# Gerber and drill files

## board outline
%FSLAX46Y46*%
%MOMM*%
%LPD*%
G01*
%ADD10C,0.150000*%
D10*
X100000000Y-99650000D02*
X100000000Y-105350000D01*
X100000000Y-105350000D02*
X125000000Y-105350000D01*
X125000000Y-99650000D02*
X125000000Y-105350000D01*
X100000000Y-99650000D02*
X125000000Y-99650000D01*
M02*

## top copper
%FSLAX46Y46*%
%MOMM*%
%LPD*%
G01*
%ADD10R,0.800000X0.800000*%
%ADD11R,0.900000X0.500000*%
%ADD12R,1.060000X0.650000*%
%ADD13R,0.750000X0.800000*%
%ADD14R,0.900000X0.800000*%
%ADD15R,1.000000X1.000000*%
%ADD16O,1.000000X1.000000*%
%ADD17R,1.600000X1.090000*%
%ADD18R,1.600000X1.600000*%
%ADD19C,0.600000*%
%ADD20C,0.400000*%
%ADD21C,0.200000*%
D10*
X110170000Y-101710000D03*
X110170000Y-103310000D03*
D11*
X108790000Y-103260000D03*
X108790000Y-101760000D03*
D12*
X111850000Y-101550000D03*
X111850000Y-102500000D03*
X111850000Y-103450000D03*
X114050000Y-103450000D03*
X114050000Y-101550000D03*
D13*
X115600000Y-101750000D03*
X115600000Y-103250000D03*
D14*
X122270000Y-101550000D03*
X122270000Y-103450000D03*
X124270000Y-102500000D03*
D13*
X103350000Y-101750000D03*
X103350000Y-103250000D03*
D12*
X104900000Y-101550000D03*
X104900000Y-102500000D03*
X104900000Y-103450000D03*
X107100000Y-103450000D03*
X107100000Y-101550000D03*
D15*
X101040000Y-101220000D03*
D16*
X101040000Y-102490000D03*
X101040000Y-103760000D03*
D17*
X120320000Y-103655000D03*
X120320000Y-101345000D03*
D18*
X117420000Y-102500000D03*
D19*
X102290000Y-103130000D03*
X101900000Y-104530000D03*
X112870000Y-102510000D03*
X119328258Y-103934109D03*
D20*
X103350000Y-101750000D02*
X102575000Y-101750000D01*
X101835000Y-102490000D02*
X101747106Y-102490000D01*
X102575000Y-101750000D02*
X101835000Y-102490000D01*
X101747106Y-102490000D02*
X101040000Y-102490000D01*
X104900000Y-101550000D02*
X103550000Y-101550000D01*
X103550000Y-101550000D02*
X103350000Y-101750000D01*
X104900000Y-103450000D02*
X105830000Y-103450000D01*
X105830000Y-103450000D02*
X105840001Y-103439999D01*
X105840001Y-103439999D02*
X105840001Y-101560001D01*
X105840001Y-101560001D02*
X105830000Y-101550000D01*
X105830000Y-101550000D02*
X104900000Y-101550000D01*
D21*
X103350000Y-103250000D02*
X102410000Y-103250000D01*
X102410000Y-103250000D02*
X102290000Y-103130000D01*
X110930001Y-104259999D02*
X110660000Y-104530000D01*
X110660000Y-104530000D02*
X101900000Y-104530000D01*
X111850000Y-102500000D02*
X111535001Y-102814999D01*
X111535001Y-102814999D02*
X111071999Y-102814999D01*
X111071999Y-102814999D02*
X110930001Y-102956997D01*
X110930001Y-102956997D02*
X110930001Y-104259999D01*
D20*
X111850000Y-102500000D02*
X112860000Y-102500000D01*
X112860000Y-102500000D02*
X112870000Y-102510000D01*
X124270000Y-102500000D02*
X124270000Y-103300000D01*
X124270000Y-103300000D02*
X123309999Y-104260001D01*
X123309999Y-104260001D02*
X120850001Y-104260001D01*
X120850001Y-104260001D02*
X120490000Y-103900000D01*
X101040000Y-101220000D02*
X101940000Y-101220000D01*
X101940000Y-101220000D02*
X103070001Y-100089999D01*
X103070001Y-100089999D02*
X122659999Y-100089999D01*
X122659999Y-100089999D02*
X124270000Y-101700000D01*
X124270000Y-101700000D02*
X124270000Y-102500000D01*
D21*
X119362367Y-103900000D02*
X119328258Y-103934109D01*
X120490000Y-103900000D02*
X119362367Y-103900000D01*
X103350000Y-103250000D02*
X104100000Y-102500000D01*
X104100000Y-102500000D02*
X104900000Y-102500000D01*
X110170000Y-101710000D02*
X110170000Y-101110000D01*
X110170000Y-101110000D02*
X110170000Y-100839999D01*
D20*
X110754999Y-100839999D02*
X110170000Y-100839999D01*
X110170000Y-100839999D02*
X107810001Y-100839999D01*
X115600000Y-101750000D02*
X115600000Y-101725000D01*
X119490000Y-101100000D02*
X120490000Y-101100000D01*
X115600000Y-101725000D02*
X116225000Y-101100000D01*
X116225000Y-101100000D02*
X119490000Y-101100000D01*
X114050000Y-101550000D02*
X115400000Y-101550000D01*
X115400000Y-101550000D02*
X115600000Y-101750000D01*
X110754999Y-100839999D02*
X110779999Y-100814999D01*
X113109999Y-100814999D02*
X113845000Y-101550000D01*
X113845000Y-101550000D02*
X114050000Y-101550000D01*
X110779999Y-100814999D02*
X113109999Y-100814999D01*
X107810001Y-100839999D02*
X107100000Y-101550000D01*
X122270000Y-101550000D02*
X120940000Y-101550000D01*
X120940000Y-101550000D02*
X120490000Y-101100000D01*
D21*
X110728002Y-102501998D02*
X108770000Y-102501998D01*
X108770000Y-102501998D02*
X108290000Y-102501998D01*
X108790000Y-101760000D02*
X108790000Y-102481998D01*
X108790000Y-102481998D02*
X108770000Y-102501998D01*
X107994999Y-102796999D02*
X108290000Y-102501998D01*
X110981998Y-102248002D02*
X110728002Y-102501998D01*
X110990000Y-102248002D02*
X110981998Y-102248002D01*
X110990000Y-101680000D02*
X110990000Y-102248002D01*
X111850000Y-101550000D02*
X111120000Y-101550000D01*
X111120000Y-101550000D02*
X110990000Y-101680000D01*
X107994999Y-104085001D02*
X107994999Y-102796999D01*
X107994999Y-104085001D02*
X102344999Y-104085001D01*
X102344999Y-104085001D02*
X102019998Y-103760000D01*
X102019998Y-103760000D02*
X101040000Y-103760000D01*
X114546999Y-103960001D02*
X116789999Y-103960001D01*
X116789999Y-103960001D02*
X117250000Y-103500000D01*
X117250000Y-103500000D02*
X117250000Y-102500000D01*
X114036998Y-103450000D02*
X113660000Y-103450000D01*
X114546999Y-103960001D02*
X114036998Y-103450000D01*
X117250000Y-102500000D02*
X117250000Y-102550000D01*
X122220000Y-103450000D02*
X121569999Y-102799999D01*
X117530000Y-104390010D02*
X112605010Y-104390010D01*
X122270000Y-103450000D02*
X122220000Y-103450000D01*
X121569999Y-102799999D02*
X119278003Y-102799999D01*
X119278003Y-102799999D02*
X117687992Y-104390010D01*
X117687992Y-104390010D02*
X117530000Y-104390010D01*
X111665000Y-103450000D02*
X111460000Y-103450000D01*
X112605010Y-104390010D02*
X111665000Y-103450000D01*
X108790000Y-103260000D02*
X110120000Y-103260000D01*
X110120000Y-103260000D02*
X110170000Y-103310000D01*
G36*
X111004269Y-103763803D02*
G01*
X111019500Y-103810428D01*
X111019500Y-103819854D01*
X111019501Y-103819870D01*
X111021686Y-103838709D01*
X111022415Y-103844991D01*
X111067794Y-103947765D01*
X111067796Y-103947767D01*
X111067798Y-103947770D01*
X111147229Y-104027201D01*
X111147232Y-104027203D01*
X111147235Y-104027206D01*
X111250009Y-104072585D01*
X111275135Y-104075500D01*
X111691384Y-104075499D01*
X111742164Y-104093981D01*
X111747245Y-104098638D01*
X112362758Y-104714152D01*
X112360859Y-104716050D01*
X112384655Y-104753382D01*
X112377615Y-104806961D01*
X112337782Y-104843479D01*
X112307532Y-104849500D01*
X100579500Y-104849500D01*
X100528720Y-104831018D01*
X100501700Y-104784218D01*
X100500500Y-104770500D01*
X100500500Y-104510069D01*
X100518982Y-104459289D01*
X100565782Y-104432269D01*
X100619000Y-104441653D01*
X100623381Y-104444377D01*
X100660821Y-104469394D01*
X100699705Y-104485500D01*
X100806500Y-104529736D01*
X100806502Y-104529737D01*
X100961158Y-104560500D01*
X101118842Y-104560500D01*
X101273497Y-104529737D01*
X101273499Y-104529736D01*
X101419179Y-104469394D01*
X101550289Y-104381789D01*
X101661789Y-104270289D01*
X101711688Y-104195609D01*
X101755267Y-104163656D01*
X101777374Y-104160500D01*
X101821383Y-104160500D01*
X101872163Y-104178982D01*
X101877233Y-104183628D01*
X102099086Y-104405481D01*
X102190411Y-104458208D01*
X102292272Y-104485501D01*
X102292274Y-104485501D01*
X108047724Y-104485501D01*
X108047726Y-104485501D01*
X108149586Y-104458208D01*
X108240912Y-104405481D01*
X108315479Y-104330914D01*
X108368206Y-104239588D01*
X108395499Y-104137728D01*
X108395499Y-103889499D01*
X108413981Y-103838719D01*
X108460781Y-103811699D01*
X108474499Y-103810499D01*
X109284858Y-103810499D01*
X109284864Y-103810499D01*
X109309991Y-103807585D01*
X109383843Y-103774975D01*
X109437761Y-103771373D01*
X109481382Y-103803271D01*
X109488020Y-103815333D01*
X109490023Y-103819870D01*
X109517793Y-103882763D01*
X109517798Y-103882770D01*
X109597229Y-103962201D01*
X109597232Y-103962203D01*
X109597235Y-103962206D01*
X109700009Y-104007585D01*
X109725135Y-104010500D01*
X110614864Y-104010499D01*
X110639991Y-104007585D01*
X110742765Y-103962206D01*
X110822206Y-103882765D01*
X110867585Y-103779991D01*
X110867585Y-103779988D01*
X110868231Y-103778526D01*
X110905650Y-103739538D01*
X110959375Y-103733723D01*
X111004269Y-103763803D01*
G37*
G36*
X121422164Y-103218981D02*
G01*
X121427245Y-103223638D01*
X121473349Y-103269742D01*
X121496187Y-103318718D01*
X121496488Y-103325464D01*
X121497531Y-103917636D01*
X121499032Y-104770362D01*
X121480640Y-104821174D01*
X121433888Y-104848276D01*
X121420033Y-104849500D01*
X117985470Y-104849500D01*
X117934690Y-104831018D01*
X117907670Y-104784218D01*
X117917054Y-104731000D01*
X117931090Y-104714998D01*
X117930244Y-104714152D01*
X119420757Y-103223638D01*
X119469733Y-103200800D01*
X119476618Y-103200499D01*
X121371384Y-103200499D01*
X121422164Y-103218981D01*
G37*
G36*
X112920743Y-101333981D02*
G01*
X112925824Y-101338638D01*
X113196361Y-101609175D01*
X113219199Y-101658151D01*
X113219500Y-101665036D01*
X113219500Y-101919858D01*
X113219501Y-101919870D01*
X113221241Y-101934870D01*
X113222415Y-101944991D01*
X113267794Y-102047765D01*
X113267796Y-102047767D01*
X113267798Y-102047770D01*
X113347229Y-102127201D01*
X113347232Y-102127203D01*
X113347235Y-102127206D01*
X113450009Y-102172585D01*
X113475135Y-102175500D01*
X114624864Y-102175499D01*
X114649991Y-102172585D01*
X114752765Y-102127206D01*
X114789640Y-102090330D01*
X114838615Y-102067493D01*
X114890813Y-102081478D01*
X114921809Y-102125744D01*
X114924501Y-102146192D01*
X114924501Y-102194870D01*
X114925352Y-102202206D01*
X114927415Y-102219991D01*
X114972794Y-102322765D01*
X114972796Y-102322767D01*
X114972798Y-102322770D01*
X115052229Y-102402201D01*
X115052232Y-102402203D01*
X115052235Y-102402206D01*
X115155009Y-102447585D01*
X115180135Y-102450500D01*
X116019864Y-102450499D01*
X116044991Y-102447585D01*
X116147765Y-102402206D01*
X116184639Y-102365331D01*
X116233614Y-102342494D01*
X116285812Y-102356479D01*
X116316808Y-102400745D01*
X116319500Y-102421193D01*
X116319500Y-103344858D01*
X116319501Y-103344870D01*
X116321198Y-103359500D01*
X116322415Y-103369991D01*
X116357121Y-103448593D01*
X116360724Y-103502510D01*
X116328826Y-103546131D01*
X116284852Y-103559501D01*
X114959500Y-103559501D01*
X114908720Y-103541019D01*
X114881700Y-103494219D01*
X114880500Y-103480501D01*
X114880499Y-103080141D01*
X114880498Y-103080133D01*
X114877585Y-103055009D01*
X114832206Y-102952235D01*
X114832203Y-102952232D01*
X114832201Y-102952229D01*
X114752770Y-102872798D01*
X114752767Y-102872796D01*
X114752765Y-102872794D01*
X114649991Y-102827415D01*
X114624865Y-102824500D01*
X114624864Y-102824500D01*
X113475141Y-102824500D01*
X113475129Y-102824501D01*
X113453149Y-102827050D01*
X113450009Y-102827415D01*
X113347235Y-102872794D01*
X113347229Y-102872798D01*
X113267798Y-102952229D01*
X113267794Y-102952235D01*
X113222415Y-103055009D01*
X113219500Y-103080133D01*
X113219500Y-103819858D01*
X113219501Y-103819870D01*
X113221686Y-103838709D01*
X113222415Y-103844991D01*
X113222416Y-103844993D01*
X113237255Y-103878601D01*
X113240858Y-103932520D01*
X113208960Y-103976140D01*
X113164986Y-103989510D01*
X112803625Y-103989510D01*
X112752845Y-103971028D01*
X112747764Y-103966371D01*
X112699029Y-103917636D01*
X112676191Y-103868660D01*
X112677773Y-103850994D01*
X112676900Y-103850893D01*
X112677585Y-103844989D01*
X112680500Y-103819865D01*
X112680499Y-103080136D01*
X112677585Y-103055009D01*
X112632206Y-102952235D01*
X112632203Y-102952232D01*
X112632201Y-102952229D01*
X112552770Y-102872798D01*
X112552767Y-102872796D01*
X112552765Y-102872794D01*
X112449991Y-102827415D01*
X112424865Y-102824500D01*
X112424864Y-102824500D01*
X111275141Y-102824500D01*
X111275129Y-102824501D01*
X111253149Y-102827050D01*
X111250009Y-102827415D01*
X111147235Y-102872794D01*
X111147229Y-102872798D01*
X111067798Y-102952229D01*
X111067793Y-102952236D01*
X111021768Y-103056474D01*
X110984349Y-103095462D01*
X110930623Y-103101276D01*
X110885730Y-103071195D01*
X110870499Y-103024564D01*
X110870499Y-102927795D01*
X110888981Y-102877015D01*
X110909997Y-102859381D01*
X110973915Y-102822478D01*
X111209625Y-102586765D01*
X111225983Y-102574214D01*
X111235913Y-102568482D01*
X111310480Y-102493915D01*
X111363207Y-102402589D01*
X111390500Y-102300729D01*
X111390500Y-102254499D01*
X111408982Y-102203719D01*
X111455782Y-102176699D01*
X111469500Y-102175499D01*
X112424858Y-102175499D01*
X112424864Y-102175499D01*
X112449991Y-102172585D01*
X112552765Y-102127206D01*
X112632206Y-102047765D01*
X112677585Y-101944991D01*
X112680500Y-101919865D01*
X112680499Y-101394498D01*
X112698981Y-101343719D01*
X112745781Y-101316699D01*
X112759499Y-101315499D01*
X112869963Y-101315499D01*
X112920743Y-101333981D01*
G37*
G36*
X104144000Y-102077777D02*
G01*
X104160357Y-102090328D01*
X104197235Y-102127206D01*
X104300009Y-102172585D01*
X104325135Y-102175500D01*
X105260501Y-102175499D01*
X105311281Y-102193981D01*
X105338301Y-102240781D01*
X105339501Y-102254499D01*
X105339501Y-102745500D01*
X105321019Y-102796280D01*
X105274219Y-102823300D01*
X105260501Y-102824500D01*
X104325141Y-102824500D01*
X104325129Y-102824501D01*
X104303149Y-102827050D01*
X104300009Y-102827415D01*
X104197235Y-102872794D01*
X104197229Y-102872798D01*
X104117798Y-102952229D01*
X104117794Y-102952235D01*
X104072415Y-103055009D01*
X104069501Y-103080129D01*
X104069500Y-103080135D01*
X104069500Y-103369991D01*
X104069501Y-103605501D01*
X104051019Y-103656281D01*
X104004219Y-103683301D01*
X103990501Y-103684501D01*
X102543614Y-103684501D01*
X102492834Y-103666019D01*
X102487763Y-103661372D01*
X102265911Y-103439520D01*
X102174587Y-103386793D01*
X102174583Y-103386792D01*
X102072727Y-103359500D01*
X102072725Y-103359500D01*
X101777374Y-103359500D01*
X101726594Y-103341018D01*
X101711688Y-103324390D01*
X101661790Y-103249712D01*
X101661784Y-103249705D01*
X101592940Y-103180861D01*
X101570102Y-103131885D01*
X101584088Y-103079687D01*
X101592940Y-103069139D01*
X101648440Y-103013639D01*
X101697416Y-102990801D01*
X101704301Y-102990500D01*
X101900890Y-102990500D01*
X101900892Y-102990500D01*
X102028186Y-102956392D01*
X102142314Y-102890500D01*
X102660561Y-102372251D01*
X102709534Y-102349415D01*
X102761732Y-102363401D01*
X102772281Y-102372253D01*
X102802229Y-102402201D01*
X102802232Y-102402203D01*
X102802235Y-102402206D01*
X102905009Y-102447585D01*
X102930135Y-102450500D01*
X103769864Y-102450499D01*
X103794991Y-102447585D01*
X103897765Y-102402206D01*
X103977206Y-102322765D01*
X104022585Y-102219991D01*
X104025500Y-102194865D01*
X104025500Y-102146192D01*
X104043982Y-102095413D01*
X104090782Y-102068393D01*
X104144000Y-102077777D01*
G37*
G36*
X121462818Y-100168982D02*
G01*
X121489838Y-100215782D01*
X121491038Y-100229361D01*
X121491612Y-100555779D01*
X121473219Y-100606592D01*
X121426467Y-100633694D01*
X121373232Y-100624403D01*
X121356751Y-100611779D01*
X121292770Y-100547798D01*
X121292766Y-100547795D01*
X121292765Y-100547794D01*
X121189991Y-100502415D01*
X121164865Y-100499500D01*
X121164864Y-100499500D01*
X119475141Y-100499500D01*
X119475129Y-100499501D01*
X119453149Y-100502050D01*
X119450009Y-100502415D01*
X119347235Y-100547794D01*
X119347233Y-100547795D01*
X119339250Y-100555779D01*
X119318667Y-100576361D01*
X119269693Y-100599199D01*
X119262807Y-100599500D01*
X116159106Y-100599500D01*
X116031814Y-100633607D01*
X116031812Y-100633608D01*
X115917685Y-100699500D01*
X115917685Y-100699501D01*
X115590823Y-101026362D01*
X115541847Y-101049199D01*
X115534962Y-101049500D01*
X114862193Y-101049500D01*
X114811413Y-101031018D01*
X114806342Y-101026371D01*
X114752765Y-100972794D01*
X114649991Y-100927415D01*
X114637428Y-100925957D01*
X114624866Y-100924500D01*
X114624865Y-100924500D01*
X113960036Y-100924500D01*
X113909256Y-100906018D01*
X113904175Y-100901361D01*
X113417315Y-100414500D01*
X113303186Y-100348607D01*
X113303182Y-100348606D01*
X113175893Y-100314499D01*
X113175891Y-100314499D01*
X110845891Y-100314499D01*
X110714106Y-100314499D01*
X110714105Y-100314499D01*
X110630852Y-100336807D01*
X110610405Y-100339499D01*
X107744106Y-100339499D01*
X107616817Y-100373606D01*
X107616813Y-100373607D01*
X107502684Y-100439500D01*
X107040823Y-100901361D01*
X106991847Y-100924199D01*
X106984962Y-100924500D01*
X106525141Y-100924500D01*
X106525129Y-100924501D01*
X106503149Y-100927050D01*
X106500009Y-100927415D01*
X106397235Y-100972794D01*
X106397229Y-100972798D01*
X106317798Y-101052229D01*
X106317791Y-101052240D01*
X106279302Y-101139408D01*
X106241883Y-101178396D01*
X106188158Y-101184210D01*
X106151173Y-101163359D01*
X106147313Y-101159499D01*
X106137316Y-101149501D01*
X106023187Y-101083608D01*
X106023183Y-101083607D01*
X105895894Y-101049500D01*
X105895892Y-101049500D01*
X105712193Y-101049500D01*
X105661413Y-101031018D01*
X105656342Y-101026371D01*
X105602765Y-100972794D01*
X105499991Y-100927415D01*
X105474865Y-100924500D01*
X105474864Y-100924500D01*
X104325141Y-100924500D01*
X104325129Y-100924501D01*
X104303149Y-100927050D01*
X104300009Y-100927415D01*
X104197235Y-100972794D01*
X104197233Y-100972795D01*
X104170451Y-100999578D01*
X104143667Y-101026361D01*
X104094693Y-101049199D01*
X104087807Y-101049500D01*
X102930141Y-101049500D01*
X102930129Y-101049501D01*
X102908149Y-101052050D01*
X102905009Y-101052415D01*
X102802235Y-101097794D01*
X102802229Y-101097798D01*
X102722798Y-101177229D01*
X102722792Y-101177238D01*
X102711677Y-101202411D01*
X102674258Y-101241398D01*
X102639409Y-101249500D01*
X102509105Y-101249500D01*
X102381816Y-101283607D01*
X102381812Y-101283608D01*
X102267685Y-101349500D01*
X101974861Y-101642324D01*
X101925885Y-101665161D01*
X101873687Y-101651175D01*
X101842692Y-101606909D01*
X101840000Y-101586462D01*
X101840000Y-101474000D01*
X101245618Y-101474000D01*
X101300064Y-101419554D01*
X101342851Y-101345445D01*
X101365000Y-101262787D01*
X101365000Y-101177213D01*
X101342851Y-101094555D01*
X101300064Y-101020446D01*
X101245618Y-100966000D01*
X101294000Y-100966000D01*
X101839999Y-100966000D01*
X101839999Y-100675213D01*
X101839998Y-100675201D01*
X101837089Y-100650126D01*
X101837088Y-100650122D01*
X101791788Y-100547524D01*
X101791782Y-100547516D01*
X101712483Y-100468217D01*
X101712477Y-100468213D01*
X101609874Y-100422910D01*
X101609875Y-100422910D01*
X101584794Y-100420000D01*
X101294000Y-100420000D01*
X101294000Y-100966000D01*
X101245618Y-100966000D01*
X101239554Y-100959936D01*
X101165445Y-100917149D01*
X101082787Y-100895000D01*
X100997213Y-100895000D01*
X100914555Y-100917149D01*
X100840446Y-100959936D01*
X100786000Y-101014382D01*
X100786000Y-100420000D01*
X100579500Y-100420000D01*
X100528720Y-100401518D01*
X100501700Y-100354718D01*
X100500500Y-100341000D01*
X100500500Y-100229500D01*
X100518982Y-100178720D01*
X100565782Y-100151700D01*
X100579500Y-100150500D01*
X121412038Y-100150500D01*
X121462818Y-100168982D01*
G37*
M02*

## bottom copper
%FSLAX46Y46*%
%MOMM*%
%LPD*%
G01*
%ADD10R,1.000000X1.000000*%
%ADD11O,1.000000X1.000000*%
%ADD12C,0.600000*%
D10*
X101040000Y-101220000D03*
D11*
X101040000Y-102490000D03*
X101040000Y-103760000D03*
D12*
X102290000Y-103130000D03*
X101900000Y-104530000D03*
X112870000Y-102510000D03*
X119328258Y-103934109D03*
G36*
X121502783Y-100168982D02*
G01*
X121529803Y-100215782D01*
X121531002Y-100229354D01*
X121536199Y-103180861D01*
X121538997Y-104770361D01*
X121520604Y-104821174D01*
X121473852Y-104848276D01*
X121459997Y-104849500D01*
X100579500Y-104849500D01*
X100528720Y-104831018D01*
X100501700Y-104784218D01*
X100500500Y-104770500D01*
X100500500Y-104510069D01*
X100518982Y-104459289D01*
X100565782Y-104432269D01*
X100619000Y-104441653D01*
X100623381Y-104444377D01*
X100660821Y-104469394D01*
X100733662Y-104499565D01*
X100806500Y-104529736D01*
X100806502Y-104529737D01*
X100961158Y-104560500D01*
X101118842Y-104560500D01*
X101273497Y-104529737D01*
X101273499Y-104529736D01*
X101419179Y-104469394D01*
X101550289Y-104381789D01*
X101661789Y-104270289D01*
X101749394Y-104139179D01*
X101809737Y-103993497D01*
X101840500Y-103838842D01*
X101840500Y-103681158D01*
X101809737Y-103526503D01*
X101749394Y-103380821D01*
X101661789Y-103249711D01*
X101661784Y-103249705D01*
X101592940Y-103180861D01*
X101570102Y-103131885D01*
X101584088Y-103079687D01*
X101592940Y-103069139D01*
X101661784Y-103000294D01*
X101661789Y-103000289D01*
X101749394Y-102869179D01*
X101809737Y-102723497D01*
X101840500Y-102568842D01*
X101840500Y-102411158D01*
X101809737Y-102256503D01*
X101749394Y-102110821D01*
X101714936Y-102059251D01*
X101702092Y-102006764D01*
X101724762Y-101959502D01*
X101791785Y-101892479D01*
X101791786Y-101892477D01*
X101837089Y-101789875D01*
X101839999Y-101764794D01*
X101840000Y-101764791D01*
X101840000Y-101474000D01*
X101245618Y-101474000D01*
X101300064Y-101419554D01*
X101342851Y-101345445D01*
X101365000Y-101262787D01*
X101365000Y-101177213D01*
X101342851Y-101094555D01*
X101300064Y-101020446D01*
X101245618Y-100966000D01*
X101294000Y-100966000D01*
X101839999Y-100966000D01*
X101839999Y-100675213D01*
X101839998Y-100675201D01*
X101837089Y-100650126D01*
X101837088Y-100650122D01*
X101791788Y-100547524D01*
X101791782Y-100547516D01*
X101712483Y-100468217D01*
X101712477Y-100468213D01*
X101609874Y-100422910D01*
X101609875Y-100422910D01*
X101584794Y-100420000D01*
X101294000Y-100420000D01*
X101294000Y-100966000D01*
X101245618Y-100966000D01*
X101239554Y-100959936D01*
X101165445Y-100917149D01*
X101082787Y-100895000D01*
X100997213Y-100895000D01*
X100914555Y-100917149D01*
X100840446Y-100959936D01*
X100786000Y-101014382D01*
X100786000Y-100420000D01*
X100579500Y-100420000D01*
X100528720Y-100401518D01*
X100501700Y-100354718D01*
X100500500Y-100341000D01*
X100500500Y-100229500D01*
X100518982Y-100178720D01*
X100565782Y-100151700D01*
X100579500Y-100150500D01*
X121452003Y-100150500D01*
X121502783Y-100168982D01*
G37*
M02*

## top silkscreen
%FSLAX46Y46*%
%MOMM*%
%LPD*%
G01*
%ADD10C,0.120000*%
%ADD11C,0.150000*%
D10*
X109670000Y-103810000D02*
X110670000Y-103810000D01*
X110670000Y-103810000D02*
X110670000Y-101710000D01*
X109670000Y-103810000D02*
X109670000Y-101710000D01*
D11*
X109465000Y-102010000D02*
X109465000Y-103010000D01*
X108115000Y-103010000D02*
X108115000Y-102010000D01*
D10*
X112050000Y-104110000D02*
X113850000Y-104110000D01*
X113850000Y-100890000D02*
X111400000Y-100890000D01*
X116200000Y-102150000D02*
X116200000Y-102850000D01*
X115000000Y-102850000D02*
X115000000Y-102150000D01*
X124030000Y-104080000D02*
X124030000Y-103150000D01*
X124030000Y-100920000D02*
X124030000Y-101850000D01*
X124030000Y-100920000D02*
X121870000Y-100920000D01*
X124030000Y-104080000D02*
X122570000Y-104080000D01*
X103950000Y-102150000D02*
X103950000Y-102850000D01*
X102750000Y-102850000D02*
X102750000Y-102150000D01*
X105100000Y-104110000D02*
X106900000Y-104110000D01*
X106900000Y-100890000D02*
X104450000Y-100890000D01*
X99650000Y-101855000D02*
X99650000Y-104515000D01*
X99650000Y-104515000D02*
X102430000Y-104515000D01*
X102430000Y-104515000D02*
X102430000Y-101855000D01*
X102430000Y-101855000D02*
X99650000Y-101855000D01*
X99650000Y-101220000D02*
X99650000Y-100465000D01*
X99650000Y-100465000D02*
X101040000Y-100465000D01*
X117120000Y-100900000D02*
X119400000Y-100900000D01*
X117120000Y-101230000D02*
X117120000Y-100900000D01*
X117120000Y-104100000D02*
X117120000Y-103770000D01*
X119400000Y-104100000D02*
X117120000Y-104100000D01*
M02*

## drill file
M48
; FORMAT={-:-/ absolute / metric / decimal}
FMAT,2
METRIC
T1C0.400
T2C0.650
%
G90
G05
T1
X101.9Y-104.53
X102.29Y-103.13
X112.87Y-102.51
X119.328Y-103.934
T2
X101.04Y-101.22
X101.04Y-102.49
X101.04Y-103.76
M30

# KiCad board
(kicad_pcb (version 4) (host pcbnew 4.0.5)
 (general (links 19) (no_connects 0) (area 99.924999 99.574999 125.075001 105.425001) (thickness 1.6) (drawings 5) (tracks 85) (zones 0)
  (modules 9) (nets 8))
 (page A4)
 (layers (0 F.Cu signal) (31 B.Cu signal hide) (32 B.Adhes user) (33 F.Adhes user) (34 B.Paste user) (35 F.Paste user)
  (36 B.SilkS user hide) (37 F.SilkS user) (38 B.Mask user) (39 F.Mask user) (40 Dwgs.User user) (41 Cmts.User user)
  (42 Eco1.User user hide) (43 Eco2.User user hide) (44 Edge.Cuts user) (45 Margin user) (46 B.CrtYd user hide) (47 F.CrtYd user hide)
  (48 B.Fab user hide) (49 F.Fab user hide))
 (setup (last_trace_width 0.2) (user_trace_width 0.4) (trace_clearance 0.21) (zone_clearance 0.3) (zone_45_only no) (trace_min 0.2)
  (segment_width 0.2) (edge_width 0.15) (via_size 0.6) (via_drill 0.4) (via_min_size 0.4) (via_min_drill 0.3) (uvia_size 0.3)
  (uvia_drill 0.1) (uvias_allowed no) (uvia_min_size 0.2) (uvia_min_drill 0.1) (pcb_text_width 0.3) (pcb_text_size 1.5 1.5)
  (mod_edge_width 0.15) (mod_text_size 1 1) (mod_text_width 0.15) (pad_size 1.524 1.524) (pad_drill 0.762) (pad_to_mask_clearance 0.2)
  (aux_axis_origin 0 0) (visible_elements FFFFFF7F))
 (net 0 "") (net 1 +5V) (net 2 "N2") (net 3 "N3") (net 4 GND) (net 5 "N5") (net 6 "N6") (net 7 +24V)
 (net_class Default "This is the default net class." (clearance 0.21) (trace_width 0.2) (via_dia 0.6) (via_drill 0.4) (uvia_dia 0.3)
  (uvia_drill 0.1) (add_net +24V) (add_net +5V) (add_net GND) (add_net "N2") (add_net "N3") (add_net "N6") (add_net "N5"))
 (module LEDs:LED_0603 (layer F.Cu) (at 110.17 102.51 90)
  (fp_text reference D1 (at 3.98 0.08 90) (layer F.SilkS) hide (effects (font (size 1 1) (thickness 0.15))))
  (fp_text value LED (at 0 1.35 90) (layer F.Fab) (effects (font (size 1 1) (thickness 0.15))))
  (fp_line (start -1.3 -0.5) (end -1.3 0.5) (layer F.SilkS) (width 0.12))
  (fp_line (start -1.3 0.5) (end 0.8 0.5) (layer F.SilkS) (width 0.12))
  (fp_line (start -1.3 -0.5) (end 0.8 -0.5) (layer F.SilkS) (width 0.12))
  (pad 2 smd rect (at 0.8 0 270) (size 0.8 0.8) (layers F.Cu F.Paste F.Mask) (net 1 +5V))
  (pad 1 smd rect (at -0.8 0 270) (size 0.8 0.8) (layers F.Cu F.Paste F.Mask) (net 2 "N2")))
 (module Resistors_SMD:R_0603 (layer F.Cu) (at 108.79 102.51 90)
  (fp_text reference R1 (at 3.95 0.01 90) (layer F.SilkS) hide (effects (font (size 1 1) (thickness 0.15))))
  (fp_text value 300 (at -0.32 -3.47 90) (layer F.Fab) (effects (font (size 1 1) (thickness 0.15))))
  (fp_line (start 0.5 0.675) (end -0.5 0.675) (layer F.SilkS) (width 0.15))
  (fp_line (start -0.5 -0.675) (end 0.5 -0.675) (layer F.SilkS) (width 0.15))
  (pad 1 smd rect (at -0.75 0 90) (size 0.5 0.9) (layers F.Cu F.Paste F.Mask) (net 2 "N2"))
  (pad 2 smd rect (at 0.75 0 90) (size 0.5 0.9) (layers F.Cu F.Paste F.Mask) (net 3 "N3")))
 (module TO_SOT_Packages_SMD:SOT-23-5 (layer F.Cu) (at 112.95 102.5)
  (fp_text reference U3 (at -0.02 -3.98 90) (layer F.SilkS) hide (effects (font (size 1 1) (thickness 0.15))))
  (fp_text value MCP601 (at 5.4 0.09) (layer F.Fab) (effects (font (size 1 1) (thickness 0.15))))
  (fp_line (start -0.9 1.61) (end 0.9 1.61) (layer F.SilkS) (width 0.12))
  (fp_line (start 0.9 -1.61) (end -1.55 -1.61) (layer F.SilkS) (width 0.12))
  (pad 1 smd rect (at -1.1 -0.95) (size 1.06 0.65) (layers F.Cu F.Paste F.Mask) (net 3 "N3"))
  (pad 2 smd rect (at -1.1 0) (size 1.06 0.65) (layers F.Cu F.Paste F.Mask) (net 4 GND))
  (pad 3 smd rect (at -1.1 0.95) (size 1.06 0.65) (layers F.Cu F.Paste F.Mask) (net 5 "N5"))
  (pad 4 smd rect (at 1.1 0.95) (size 1.06 0.65) (layers F.Cu F.Paste F.Mask) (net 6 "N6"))
  (pad 5 smd rect (at 1.1 -0.95) (size 1.06 0.65) (layers F.Cu F.Paste F.Mask) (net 1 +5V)))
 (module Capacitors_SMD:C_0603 (layer F.Cu) (at 115.6 102.5 270)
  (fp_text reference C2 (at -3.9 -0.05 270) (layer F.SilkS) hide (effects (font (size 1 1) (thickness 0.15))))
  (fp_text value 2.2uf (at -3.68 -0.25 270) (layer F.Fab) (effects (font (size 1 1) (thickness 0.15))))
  (fp_line (start -0.35 -0.6) (end 0.35 -0.6) (layer F.SilkS) (width 0.12))
  (fp_line (start 0.35 0.6) (end -0.35 0.6) (layer F.SilkS) (width 0.12))
  (pad 1 smd rect (at -0.75 0 270) (size 0.8 0.75) (layers F.Cu F.Paste F.Mask) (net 1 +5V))
  (pad 2 smd rect (at 0.75 0 270) (size 0.8 0.75) (layers F.Cu F.Paste F.Mask) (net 4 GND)))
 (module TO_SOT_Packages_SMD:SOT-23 (layer F.Cu) (at 123.27 102.5)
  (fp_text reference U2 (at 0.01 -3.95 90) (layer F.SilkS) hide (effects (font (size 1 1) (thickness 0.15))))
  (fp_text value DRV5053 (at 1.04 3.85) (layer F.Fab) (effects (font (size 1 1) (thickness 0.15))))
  (fp_line (start 0.76 1.58) (end 0.76 0.65) (layer F.SilkS) (width 0.12))
  (fp_line (start 0.76 -1.58) (end 0.76 -0.65) (layer F.SilkS) (width 0.12))
  (fp_line (start 0.76 -1.58) (end -1.4 -1.58) (layer F.SilkS) (width 0.12))
  (fp_line (start 0.76 1.58) (end -0.7 1.58) (layer F.SilkS) (width 0.12))
  (pad 1 smd rect (at -1 -0.95) (size 0.9 0.8) (layers F.Cu F.Paste F.Mask) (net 1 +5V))
  (pad 2 smd rect (at -1 0.95) (size 0.9 0.8) (layers F.Cu F.Paste F.Mask) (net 5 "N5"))
  (pad 3 smd rect (at 1 0) (size 0.9 0.8) (layers F.Cu F.Paste F.Mask) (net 4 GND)))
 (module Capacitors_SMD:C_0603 (layer F.Cu) (at 103.35 102.5 270)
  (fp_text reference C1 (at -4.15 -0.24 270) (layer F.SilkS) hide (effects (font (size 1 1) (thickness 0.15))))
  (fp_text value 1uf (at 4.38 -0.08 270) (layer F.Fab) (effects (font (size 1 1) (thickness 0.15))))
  (fp_line (start -0.35 -0.6) (end 0.35 -0.6) (layer F.SilkS) (width 0.12))
  (fp_line (start 0.35 0.6) (end -0.35 0.6) (layer F.SilkS) (width 0.12))
  (pad 1 smd rect (at -0.75 0 270) (size 0.8 0.75) (layers F.Cu F.Paste F.Mask) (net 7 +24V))
  (pad 2 smd rect (at 0.75 0 270) (size 0.8 0.75) (layers F.Cu F.Paste F.Mask) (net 4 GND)))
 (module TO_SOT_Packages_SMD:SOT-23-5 (layer F.Cu) (at 106 102.5)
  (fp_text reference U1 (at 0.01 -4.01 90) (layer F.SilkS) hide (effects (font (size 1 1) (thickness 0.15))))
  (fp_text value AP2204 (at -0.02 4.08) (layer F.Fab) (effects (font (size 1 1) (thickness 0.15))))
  (fp_line (start -0.9 1.61) (end 0.9 1.61) (layer F.SilkS) (width 0.12))
  (fp_line (start 0.9 -1.61) (end -1.55 -1.61) (layer F.SilkS) (width 0.12))
  (pad 1 smd rect (at -1.1 -0.95) (size 1.06 0.65) (layers F.Cu F.Paste F.Mask) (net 7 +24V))
  (pad 2 smd rect (at -1.1 0) (size 1.06 0.65) (layers F.Cu F.Paste F.Mask) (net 4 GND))
  (pad 3 smd rect (at -1.1 0.95) (size 1.06 0.65) (layers F.Cu F.Paste F.Mask) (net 7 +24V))
  (pad 4 smd rect (at 1.1 0.95) (size 1.06 0.65) (layers F.Cu F.Paste F.Mask))
  (pad 5 smd rect (at 1.1 -0.95) (size 1.06 0.65) (layers F.Cu F.Paste F.Mask) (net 1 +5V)))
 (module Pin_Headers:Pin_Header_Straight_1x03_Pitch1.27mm (layer F.Cu) (at 101.04 101.22)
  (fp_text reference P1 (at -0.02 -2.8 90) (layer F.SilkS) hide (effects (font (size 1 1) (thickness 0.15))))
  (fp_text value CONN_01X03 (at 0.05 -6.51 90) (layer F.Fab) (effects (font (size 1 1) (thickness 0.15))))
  (fp_line (start -1.39 0.635) (end -1.39 3.295) (layer F.SilkS) (width 0.12))
  (fp_line (start -1.39 3.295) (end 1.39 3.295) (layer F.SilkS) (width 0.12))
  (fp_line (start 1.39 3.295) (end 1.39 0.635) (layer F.SilkS) (width 0.12))
  (fp_line (start 1.39 0.635) (end -1.39 0.635) (layer F.SilkS) (width 0.12))
  (fp_line (start -1.39 0) (end -1.39 -0.755) (layer F.SilkS) (width 0.12))
  (fp_line (start -1.39 -0.755) (end 0 -0.755) (layer F.SilkS) (width 0.12))
  (pad 1 thru_hole rect (at 0 0) (size 1 1) (drill 0.65) (layers *.Cu *.Mask) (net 4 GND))
  (pad 2 thru_hole oval (at 0 1.27) (size 1 1) (drill 0.65) (layers *.Cu *.Mask) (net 7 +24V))
  (pad 3 thru_hole oval (at 0 2.54) (size 1 1) (drill 0.65) (layers *.Cu *.Mask) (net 3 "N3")))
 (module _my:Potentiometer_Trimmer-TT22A (layer F.Cu) (at 118.87 102.5 90)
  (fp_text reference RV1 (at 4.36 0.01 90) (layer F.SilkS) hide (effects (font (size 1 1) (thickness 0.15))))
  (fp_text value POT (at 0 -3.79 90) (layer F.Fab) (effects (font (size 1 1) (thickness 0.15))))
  (fp_line (start 1.6 -1.75) (end 1.6 0.53) (layer F.SilkS) (width 0.12))
  (fp_line (start 1.27 -1.75) (end 1.6 -1.75) (layer F.SilkS) (width 0.12))
  (fp_line (start -1.6 -1.75) (end -1.27 -1.75) (layer F.SilkS) (width 0.12))
  (fp_line (start -1.6 0.53) (end -1.6 -1.75) (layer F.SilkS) (width 0.12))
  (pad 1 smd rect (at -1.155 1.45 90) (size 1.09 1.6) (layers F.Cu F.Paste F.Mask) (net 4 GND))
  (pad 3 smd rect (at 1.155 1.45 90) (size 1.09 1.6) (layers F.Cu F.Paste F.Mask) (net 1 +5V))
  (pad 2 smd rect (at 0 -1.45 90) (size 1.6 1.6) (layers F.Cu F.Paste F.Mask) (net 6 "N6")))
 (gr_line (start 100 99.65) (end 100 105.35) (layer Edge.Cuts) (width 0.15))
 (gr_line (start 100 105.35) (end 125 105.35) (layer Edge.Cuts) (width 0.15))
 (gr_line (start 125 99.65) (end 125 105.35) (layer Edge.Cuts) (width 0.15))
 (gr_line (start 100 99.65) (end 125 99.65) (layer Edge.Cuts) (width 0.15))
 (segment (start 103.35 101.75) (end 102.575 101.75) (width 0.4) (layer F.Cu) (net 7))
 (segment (start 101.835 102.49) (end 101.747106 102.49) (width 0.4) (layer F.Cu) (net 7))
 (segment (start 102.575 101.75) (end 101.835 102.49) (width 0.4) (layer F.Cu) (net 7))
 (segment (start 101.747106 102.49) (end 101.04 102.49) (width 0.4) (layer F.Cu) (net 7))
 (segment (start 104.9 101.55) (end 103.55 101.55) (width 0.4) (layer F.Cu) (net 7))
 (segment (start 103.55 101.55) (end 103.35 101.75) (width 0.4) (layer F.Cu) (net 7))
 (segment (start 104.9 103.45) (end 105.83 103.45) (width 0.4) (layer F.Cu) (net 7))
 (segment (start 105.83 103.45) (end 105.840001 103.439999) (width 0.4) (layer F.Cu) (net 7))
 (segment (start 105.840001 103.439999) (end 105.840001 101.560001) (width 0.4) (layer F.Cu) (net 7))
 (segment (start 105.840001 101.560001) (end 105.83 101.55) (width 0.4) (layer F.Cu) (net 7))
 (segment (start 105.83 101.55) (end 104.9 101.55) (width 0.4) (layer F.Cu) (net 7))
 (segment (start 103.35 103.25) (end 102.41 103.25) (width 0.2) (layer F.Cu) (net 4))
 (via (at 102.29 103.13) (size 0.6) (drill 0.4) (layers F.Cu B.Cu) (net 4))
 (segment (start 102.41 103.25) (end 102.29 103.13) (width 0.2) (layer F.Cu) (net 4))
 (segment (start 110.930001 104.259999) (end 110.66 104.53) (width 0.2) (layer F.Cu) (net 4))
 (segment (start 110.66 104.53) (end 101.9 104.53) (width 0.2) (layer F.Cu) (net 4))
 (via (at 101.9 104.53) (size 0.6) (drill 0.4) (layers F.Cu B.Cu) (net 4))
 (segment (start 111.85 102.5) (end 111.535001 102.814999) (width 0.2) (layer F.Cu) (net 4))
 (segment (start 111.535001 102.814999) (end 111.071999 102.814999) (width 0.2) (layer F.Cu) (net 4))
 (segment (start 111.071999 102.814999) (end 110.930001 102.956997) (width 0.2) (layer F.Cu) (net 4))
 (segment (start 110.930001 102.956997) (end 110.930001 104.259999) (width 0.2) (layer F.Cu) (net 4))
 (segment (start 111.85 102.5) (end 112.86 102.5) (width 0.4) (layer F.Cu) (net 4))
 (segment (start 112.86 102.5) (end 112.87 102.51) (width 0.4) (layer F.Cu) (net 4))
 (via (at 112.87 102.51) (size 0.6) (drill 0.4) (layers F.Cu B.Cu) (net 4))
 (segment (start 124.27 102.5) (end 124.27 103.3) (width 0.4) (layer F.Cu) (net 4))
 (segment (start 124.27 103.3) (end 123.309999 104.260001) (width 0.4) (layer F.Cu) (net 4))
 (segment (start 123.309999 104.260001) (end 120.850001 104.260001) (width 0.4) (layer F.Cu) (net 4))
 (segment (start 120.850001 104.260001) (end 120.49 103.9) (width 0.4) (layer F.Cu) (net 4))
 (segment (start 101.04 101.22) (end 101.94 101.22) (width 0.4) (layer F.Cu) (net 4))
 (segment (start 101.94 101.22) (end 103.070001 100.089999) (width 0.4) (layer F.Cu) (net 4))
 (segment (start 103.070001 100.089999) (end 122.659999 100.089999) (width 0.4) (layer F.Cu) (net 4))
 (segment (start 122.659999 100.089999) (end 124.27 101.7) (width 0.4) (layer F.Cu) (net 4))
 (segment (start 124.27 101.7) (end 124.27 102.5) (width 0.4) (layer F.Cu) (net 4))
 (segment (start 119.362367 103.9) (end 119.328258 103.934109) (width 0.2) (layer F.Cu) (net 4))
 (segment (start 120.49 103.9) (end 119.362367 103.9) (width 0.2) (layer F.Cu) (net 4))
 (via (at 119.328258 103.934109) (size 0.6) (drill 0.4) (layers F.Cu B.Cu) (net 4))
 (segment (start 103.35 103.25) (end 104.1 102.5) (width 0.2) (layer F.Cu) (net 4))
 (segment (start 104.1 102.5) (end 104.9 102.5) (width 0.2) (layer F.Cu) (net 4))
 (segment (start 110.17 101.71) (end 110.17 101.11) (width 0.2) (layer F.Cu) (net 1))
 (segment (start 110.17 101.11) (end 110.17 100.839999) (width 0.2) (layer F.Cu) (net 1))
 (segment (start 110.754999 100.839999) (end 110.17 100.839999) (width 0.4) (layer F.Cu) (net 1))
 (segment (start 110.17 100.839999) (end 107.810001 100.839999) (width 0.4) (layer F.Cu) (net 1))
 (segment (start 115.6 101.75) (end 115.6 101.725) (width 0.4) (layer F.Cu) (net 1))
 (segment (start 119.49 101.1) (end 120.49 101.1) (width 0.4) (layer F.Cu) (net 1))
 (segment (start 115.6 101.725) (end 116.225 101.1) (width 0.4) (layer F.Cu) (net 1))
 (segment (start 116.225 101.1) (end 119.49 101.1) (width 0.4) (layer F.Cu) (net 1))
 (segment (start 114.05 101.55) (end 115.4 101.55) (width 0.4) (layer F.Cu) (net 1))
 (segment (start 115.4 101.55) (end 115.6 101.75) (width 0.4) (layer F.Cu) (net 1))
 (segment (start 110.754999 100.839999) (end 110.779999 100.814999) (width 0.4) (layer F.Cu) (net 1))
 (segment (start 113.109999 100.814999) (end 113.845 101.55) (width 0.4) (layer F.Cu) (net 1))
 (segment (start 113.845 101.55) (end 114.05 101.55) (width 0.4) (layer F.Cu) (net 1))
 (segment (start 110.779999 100.814999) (end 113.109999 100.814999) (width 0.4) (layer F.Cu) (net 1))
 (segment (start 107.810001 100.839999) (end 107.1 101.55) (width 0.4) (layer F.Cu) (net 1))
 (segment (start 122.27 101.55) (end 120.94 101.55) (width 0.4) (layer F.Cu) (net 1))
 (segment (start 120.94 101.55) (end 120.49 101.1) (width 0.4) (layer F.Cu) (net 1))
 (segment (start 110.728002 102.501998) (end 108.77 102.501998) (width 0.2) (layer F.Cu) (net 3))
 (segment (start 108.77 102.501998) (end 108.29 102.501998) (width 0.2) (layer F.Cu) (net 3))
 (segment (start 108.79 101.76) (end 108.79 102.481998) (width 0.2) (layer F.Cu) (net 3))
 (segment (start 108.79 102.481998) (end 108.77 102.501998) (width 0.2) (layer F.Cu) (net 3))
 (segment (start 107.994999 102.796999) (end 108.29 102.501998) (width 0.2) (layer F.Cu) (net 3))
 (segment (start 110.981998 102.248002) (end 110.728002 102.501998) (width 0.2) (layer F.Cu) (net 3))
 (segment (start 110.99 102.248002) (end 110.981998 102.248002) (width 0.2) (layer F.Cu) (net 3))
 (segment (start 110.99 101.68) (end 110.99 102.248002) (width 0.2) (layer F.Cu) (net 3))
 (segment (start 111.85 101.55) (end 111.12 101.55) (width 0.2) (layer F.Cu) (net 3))
 (segment (start 111.12 101.55) (end 110.99 101.68) (width 0.2) (layer F.Cu) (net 3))
 (segment (start 107.994999 104.085001) (end 107.994999 102.796999) (width 0.2) (layer F.Cu) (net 3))
 (segment (start 107.994999 104.085001) (end 102.344999 104.085001) (width 0.2) (layer F.Cu) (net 3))
 (segment (start 102.344999 104.085001) (end 102.019998 103.76) (width 0.2) (layer F.Cu) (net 3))
 (segment (start 102.019998 103.76) (end 101.04 103.76) (width 0.2) (layer F.Cu) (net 3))
 (segment (start 114.546999 103.960001) (end 116.789999 103.960001) (width 0.2) (layer F.Cu) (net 6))
 (segment (start 116.789999 103.960001) (end 117.25 103.5) (width 0.2) (layer F.Cu) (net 6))
 (segment (start 117.25 103.5) (end 117.25 102.5) (width 0.2) (layer F.Cu) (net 6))
 (segment (start 114.036998 103.45) (end 113.66 103.45) (width 0.2) (layer F.Cu) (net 6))
 (segment (start 114.546999 103.960001) (end 114.036998 103.45) (width 0.2) (layer F.Cu) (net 6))
 (segment (start 117.25 102.5) (end 117.25 102.55) (width 0.2) (layer F.Cu) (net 6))
 (segment (start 122.22 103.45) (end 121.569999 102.799999) (width 0.2) (layer F.Cu) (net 5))
 (segment (start 117.53 104.39001) (end 112.60501 104.39001) (width 0.2) (layer F.Cu) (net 5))
 (segment (start 122.27 103.45) (end 122.22 103.45) (width 0.2) (layer F.Cu) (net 5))
 (segment (start 121.569999 102.799999) (end 119.278003 102.799999) (width 0.2) (layer F.Cu) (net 5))
 (segment (start 119.278003 102.799999) (end 117.687992 104.39001) (width 0.2) (layer F.Cu) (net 5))
 (segment (start 117.687992 104.39001) (end 117.53 104.39001) (width 0.2) (layer F.Cu) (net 5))
 (segment (start 111.665 103.45) (end 111.46 103.45) (width 0.2) (layer F.Cu) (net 5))
 (segment (start 112.60501 104.39001) (end 111.665 103.45) (width 0.2) (layer F.Cu) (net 5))
 (segment (start 108.79 103.26) (end 110.12 103.26) (width 0.2) (layer F.Cu) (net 2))
 (segment (start 110.12 103.26) (end 110.17 103.31) (width 0.2) (layer F.Cu) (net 2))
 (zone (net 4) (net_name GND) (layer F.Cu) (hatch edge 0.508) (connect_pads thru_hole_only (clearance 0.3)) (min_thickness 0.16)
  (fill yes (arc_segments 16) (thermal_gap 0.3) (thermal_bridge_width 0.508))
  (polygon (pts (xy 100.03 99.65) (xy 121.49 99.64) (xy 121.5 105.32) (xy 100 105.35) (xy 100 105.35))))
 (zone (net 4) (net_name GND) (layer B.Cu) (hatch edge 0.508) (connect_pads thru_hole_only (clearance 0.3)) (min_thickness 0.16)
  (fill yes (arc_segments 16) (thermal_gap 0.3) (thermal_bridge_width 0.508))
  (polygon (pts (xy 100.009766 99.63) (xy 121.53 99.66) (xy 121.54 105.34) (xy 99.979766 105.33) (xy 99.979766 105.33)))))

